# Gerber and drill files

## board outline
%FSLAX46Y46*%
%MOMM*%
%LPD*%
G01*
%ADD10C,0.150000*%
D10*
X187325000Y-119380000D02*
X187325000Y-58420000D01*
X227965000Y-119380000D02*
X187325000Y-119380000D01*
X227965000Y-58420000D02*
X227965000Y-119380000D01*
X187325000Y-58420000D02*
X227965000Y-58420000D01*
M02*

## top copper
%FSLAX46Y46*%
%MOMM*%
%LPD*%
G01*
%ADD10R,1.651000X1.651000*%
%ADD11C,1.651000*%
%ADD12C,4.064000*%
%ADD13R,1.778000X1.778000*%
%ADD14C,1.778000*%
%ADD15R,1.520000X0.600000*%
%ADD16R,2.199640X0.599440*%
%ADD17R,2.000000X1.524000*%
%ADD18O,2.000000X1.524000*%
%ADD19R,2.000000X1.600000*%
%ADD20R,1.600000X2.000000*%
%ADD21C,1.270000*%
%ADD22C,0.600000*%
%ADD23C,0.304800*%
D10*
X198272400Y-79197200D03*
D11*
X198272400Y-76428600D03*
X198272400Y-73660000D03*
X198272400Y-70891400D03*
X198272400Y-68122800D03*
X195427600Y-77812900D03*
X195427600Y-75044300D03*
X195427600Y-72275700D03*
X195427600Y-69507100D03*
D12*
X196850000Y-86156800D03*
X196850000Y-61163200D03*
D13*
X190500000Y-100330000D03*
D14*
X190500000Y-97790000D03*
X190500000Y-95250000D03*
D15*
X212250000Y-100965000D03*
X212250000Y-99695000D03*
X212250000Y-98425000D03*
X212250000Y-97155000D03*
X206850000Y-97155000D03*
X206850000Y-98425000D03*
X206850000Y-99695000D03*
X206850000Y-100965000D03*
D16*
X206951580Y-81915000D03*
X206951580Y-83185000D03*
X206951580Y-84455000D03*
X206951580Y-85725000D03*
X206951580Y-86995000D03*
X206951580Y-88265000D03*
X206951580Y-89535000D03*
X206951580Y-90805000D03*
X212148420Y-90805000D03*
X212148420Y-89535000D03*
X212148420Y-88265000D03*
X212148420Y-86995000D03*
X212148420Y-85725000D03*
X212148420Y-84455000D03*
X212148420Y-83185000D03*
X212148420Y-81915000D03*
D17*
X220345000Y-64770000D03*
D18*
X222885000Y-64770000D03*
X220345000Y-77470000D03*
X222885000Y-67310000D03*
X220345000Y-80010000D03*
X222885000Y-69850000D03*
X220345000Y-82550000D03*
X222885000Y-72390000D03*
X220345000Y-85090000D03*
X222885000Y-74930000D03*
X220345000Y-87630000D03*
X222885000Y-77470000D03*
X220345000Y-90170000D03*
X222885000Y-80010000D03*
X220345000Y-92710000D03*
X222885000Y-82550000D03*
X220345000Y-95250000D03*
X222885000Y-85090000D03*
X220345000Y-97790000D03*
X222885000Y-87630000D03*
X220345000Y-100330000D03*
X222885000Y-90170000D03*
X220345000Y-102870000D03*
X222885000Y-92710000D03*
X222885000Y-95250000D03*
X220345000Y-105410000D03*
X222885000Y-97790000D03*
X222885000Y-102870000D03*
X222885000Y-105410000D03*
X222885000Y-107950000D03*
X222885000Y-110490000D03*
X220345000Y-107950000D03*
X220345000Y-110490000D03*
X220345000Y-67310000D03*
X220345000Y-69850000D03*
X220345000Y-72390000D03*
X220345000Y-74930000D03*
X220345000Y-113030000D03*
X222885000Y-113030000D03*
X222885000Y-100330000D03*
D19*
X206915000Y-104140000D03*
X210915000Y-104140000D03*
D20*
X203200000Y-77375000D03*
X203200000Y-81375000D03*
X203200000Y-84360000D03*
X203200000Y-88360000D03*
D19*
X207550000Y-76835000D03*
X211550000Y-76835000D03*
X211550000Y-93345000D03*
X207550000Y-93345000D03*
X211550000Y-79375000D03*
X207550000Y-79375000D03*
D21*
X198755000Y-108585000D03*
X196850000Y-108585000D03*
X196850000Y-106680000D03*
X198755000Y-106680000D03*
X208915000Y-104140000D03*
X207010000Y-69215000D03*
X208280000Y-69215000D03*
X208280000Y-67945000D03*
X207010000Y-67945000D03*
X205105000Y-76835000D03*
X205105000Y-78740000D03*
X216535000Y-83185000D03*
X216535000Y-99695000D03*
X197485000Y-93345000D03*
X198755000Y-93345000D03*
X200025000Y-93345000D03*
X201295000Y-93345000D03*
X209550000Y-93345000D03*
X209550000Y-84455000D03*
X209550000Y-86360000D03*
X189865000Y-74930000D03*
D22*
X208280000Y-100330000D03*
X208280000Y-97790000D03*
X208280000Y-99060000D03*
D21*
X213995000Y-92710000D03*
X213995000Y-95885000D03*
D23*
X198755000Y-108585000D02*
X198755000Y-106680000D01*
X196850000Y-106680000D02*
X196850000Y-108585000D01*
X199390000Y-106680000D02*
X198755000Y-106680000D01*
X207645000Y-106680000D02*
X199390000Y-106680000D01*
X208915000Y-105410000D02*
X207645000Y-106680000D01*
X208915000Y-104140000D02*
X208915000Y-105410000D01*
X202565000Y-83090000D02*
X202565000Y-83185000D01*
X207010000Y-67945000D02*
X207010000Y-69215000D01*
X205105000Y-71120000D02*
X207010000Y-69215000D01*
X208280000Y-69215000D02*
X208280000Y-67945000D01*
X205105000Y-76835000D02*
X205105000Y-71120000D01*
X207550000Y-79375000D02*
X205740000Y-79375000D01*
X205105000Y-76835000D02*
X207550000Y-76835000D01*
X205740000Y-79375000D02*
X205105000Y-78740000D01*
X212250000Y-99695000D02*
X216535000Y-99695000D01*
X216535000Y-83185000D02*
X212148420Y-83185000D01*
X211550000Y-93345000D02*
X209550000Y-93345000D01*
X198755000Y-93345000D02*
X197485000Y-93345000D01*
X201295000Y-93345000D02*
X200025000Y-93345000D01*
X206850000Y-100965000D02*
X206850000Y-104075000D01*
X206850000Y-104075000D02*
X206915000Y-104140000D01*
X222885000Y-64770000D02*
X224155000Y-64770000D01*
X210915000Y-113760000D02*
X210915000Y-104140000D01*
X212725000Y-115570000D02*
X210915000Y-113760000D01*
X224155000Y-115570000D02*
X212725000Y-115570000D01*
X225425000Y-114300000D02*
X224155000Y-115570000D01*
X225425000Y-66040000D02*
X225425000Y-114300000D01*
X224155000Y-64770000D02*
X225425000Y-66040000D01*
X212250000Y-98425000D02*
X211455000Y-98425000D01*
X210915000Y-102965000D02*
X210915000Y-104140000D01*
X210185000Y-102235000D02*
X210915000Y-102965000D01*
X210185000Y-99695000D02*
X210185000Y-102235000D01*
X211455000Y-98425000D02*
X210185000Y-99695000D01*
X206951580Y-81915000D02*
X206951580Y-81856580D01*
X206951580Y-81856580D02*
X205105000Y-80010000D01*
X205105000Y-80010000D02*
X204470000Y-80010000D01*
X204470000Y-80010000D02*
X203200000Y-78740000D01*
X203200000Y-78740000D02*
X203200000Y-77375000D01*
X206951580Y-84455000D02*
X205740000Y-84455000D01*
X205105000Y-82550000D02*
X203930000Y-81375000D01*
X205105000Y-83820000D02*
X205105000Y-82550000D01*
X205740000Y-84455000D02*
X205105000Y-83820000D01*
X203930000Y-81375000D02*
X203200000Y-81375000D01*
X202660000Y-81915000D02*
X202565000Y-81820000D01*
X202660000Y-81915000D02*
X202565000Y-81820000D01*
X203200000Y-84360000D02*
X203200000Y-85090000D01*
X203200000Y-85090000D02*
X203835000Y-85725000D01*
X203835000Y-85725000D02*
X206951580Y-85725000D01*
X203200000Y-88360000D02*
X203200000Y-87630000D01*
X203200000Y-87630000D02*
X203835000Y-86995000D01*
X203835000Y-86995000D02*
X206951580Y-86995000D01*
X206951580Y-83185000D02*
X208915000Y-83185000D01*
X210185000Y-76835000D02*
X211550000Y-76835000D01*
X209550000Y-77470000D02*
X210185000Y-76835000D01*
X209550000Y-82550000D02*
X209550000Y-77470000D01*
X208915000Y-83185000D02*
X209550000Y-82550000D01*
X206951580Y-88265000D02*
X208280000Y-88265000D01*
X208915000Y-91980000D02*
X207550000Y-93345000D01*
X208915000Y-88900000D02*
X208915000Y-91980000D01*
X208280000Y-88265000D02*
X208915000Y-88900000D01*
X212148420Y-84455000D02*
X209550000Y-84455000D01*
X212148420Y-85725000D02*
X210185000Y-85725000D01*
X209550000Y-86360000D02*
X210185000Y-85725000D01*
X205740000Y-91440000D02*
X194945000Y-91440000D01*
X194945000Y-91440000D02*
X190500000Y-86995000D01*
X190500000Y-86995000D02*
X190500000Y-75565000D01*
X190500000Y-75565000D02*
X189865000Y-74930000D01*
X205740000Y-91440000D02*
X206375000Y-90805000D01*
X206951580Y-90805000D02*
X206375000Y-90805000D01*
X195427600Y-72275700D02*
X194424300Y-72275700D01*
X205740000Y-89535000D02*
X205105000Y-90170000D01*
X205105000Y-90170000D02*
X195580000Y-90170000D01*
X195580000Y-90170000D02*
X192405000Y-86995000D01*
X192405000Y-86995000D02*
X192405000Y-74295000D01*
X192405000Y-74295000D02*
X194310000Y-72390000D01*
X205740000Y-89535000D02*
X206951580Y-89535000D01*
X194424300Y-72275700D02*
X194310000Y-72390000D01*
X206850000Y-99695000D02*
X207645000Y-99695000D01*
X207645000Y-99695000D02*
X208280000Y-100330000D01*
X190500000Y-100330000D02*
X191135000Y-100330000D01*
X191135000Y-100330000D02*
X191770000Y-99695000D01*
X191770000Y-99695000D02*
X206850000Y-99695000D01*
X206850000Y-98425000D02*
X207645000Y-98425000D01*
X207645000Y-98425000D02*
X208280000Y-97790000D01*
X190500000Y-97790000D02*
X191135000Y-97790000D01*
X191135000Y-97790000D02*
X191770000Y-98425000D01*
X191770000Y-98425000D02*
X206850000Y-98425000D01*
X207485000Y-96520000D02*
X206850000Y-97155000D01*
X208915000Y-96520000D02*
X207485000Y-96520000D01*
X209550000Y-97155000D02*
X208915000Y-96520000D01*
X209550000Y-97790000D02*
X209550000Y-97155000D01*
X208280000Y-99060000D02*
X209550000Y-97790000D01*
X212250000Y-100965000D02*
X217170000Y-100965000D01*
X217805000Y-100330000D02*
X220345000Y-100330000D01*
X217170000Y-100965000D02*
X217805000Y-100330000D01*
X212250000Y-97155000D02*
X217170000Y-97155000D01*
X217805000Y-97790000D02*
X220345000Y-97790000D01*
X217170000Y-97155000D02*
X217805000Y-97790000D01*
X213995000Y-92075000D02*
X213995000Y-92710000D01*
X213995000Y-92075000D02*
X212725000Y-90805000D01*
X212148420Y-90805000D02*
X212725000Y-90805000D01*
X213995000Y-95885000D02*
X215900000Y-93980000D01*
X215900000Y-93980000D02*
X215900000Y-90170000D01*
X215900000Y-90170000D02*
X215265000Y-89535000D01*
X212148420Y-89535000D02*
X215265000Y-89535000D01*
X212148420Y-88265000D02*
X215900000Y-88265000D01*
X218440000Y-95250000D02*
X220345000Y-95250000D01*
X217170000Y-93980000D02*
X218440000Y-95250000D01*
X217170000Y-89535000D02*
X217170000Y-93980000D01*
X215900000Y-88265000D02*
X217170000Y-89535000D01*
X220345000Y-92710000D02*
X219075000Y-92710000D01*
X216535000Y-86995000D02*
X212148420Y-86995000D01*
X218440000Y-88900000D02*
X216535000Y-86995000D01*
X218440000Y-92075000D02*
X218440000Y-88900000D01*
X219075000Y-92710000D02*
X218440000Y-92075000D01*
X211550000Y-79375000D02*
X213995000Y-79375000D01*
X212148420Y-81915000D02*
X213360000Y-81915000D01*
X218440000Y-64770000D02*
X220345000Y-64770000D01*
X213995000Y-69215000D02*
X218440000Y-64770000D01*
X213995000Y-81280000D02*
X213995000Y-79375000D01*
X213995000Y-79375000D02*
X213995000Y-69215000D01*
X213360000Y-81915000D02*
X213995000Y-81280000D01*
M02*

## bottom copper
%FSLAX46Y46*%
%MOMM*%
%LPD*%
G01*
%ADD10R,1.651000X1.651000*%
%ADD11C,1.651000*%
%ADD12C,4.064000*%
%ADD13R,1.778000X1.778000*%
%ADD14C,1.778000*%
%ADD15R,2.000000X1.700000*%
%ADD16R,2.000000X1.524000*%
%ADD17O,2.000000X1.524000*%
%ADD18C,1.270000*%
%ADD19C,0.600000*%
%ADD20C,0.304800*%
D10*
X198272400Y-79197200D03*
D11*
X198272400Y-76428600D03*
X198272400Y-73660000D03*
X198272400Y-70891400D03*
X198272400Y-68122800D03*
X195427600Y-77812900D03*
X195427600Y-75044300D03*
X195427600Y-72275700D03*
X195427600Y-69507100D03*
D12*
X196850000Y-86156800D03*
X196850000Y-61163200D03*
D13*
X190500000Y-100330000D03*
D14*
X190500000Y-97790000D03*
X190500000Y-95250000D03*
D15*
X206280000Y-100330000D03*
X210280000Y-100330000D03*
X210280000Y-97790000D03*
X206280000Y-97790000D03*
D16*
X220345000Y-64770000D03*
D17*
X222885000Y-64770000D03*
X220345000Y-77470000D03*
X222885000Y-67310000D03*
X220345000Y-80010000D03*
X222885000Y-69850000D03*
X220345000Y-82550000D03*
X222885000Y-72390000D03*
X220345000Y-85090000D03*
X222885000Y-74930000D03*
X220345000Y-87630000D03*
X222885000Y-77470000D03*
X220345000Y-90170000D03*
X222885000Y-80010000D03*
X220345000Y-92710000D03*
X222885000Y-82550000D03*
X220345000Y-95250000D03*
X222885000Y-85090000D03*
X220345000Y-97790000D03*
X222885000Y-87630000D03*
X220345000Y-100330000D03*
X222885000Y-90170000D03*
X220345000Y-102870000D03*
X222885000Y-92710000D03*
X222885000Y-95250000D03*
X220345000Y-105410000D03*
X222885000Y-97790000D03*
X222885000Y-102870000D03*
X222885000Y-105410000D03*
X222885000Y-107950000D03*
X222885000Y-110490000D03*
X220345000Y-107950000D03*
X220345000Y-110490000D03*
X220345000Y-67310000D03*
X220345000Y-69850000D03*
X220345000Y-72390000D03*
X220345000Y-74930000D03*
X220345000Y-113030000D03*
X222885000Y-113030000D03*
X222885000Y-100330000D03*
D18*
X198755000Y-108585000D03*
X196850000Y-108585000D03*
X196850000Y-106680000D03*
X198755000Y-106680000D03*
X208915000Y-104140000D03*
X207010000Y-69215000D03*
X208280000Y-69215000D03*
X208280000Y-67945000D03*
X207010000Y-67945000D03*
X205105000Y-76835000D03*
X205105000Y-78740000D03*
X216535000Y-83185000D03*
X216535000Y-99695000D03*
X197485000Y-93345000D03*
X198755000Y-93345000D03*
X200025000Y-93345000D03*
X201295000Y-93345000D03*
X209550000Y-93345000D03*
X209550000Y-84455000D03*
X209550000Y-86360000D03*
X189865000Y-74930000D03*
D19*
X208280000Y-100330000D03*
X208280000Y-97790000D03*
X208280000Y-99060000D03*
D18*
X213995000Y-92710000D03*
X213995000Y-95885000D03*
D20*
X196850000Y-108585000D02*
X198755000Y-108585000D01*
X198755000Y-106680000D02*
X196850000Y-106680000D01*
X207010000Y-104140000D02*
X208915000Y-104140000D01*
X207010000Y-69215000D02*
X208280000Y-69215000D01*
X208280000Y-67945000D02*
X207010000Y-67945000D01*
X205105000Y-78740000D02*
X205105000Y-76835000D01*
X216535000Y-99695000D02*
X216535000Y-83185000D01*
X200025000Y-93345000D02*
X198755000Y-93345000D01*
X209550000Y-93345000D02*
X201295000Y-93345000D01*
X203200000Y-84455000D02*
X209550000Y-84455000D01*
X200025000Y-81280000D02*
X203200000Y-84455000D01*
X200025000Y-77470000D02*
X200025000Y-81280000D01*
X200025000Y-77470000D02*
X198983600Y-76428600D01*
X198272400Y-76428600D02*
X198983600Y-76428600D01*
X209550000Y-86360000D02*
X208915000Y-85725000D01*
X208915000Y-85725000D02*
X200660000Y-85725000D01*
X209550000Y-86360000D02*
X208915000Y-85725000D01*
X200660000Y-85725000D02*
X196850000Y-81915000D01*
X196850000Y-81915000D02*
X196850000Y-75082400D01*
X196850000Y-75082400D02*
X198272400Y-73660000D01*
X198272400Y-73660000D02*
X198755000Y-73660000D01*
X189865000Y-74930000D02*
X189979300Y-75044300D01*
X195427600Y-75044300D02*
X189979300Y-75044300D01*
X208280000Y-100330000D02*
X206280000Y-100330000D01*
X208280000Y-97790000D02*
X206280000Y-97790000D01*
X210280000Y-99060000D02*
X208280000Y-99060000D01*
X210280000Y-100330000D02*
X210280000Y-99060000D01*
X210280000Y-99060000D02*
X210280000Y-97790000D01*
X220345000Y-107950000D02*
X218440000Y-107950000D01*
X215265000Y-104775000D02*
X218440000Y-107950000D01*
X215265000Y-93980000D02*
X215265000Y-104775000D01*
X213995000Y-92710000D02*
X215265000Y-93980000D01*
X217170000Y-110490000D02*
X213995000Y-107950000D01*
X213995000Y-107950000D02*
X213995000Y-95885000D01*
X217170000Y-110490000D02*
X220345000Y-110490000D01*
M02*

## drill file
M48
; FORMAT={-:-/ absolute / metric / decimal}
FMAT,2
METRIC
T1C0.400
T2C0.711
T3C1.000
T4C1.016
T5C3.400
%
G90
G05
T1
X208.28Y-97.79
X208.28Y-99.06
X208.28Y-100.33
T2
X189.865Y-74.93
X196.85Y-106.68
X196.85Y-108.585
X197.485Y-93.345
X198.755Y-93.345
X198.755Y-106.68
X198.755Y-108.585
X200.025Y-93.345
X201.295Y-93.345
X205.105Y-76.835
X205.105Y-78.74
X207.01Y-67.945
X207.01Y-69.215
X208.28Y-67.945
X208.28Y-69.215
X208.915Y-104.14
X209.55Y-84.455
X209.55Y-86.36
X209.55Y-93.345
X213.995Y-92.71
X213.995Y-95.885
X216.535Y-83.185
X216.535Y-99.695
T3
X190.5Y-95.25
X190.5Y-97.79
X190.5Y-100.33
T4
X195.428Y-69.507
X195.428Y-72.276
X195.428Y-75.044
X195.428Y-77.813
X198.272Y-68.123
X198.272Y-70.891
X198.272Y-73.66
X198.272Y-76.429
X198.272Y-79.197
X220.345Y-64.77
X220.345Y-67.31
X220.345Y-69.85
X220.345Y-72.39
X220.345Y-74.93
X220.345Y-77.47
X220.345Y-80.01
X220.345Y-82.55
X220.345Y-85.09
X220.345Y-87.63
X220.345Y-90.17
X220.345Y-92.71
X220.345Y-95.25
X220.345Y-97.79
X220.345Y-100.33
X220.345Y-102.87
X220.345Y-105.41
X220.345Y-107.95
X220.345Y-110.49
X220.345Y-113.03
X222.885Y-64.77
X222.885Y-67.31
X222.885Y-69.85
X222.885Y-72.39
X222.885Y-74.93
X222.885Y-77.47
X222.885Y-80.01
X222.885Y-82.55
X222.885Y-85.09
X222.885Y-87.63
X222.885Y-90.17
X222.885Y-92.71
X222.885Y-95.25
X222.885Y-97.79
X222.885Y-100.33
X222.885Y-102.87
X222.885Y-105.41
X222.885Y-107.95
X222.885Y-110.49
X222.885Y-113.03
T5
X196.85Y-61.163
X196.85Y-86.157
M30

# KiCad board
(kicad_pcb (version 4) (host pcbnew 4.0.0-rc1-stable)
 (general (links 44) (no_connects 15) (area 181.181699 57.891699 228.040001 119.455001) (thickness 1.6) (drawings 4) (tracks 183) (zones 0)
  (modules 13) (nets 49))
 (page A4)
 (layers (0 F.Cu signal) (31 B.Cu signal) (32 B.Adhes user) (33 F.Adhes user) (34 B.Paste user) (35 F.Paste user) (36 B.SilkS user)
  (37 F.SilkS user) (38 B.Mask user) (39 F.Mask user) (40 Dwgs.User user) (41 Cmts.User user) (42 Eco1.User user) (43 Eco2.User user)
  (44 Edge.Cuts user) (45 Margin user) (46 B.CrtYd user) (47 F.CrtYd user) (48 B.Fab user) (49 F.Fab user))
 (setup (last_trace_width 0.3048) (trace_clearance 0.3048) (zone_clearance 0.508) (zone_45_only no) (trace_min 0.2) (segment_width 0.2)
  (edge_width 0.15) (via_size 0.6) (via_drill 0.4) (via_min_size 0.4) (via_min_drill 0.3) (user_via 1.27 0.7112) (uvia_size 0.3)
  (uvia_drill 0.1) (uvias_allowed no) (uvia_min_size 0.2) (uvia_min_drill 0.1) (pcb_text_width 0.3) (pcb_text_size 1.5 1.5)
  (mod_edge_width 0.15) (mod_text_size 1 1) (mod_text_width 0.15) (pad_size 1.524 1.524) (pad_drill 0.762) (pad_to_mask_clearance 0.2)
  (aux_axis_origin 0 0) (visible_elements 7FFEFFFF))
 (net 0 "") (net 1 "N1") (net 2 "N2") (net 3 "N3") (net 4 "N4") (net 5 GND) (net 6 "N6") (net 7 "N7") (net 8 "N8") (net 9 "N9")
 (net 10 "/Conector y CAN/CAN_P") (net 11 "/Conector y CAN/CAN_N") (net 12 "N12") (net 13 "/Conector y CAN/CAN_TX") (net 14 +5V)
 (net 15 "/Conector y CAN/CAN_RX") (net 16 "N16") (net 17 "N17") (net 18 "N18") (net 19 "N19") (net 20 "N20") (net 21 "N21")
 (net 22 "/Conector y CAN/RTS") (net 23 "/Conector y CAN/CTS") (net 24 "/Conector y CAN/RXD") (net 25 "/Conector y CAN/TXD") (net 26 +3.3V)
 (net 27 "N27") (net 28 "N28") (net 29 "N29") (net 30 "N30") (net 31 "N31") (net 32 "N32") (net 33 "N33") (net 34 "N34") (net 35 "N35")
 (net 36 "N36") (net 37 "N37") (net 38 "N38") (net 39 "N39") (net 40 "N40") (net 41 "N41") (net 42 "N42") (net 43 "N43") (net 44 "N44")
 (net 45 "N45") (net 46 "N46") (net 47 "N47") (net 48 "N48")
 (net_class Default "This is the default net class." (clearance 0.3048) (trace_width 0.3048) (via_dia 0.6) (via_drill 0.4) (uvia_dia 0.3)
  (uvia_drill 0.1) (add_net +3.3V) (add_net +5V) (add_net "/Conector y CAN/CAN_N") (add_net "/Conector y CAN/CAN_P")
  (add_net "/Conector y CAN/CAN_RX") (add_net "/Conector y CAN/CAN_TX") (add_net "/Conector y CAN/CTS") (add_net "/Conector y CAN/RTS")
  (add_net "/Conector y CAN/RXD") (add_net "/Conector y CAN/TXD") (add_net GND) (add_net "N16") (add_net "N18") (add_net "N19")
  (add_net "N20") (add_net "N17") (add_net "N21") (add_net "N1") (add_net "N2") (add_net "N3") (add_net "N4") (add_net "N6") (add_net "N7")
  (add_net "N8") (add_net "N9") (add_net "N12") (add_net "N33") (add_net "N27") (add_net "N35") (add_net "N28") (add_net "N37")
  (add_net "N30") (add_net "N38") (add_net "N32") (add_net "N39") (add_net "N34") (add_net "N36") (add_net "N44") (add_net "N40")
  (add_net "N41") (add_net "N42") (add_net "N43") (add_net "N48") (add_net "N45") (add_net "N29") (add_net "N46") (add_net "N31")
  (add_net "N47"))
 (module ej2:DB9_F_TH (layer F.Cu) (at 196.85 73.66 90)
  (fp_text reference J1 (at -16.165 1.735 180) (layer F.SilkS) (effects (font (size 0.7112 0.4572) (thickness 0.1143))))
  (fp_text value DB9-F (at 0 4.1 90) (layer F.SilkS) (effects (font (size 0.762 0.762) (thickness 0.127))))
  (pad 1 thru_hole rect (at -5.5372 1.4224 90) (size 1.651 1.651) (drill 1.016) (layers *.Cu *.Mask) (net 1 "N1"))
  (pad 2 thru_hole circle (at -2.7686 1.4224 90) (size 1.651 1.651) (drill 1.016) (layers *.Cu *.Mask) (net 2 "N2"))
  (pad 3 thru_hole circle (at 0 1.4224 90) (size 1.651 1.651) (drill 1.016) (layers *.Cu *.Mask) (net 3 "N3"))
  (pad 4 thru_hole circle (at 2.7686 1.4224 90) (size 1.651 1.651) (drill 1.016) (layers *.Cu *.Mask) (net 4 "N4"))
  (pad 5 thru_hole circle (at 5.5372 1.4224 90) (size 1.651 1.651) (drill 1.016) (layers *.Cu *.Mask) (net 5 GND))
  (pad 6 thru_hole circle (at -4.1529 -1.4224 90) (size 1.651 1.651) (drill 1.016) (layers *.Cu *.Mask) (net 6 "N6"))
  (pad 7 thru_hole circle (at -1.3843 -1.4224 90) (size 1.651 1.651) (drill 1.016) (layers *.Cu *.Mask) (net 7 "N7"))
  (pad 8 thru_hole circle (at 1.3843 -1.4224 90) (size 1.651 1.651) (drill 1.016) (layers *.Cu *.Mask) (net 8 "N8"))
  (pad 9 thru_hole circle (at 4.1529 -1.4224 90) (size 1.651 1.651) (drill 1.016) (layers *.Cu *.Mask) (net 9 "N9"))
  (pad 10 thru_hole circle (at -12.4968 0 90) (size 4.064 4.064) (drill 3.4) (layers *.Cu *.Mask))
  (pad 11 thru_hole circle (at 12.4968 0 90) (size 4.064 4.064) (drill 3.4) (layers *.Cu *.Mask)))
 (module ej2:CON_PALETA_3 (layer F.Cu) (at 190.5 97.79 90)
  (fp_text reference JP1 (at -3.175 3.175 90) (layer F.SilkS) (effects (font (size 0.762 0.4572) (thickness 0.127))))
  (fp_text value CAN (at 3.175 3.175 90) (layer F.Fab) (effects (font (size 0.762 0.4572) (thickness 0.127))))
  (pad 1 thru_hole rect (at -2.54 0 90) (size 1.778 1.778) (drill 1) (layers *.Cu *.Mask) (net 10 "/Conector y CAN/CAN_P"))
  (pad 2 thru_hole circle (at 0 0 90) (size 1.778 1.778) (drill 1) (layers *.Cu *.Mask) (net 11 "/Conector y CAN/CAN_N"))
  (pad 3 thru_hole circle (at 2.54 0 90) (size 1.778 1.778) (drill 1) (layers *.Cu *.Mask) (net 5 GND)))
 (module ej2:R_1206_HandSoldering (layer B.Cu) (at 208.28 100.33)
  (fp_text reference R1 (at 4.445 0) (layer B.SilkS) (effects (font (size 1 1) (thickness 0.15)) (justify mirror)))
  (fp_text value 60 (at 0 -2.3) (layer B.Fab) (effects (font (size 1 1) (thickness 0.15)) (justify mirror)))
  (pad 1 smd rect (at -2 0) (size 2 1.7) (layers B.Cu B.Paste B.Mask) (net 10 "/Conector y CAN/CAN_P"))
  (pad 2 smd rect (at 2 0) (size 2 1.7) (layers B.Cu B.Paste B.Mask) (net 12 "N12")))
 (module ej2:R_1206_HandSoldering (layer B.Cu) (at 208.28 97.79 180)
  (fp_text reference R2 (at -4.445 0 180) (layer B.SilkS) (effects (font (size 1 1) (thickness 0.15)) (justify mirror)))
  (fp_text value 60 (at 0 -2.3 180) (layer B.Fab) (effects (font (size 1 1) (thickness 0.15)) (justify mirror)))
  (pad 1 smd rect (at -2 0 180) (size 2 1.7) (layers B.Cu B.Paste B.Mask) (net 12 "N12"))
  (pad 2 smd rect (at 2 0 180) (size 2 1.7) (layers B.Cu B.Paste B.Mask) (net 11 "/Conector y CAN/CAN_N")))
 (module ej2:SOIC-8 (layer F.Cu) (at 209.55 99.06 180)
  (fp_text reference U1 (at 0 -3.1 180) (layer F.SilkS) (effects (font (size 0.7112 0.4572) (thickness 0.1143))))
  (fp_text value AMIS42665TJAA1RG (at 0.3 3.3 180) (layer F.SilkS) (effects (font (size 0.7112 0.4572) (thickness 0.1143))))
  (pad 1 smd rect (at -2.7 -1.905 90) (size 0.6 1.52) (layers F.Cu F.Paste F.Mask) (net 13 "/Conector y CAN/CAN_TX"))
  (pad 2 smd rect (at -2.7 -0.635 90) (size 0.6 1.52) (layers F.Cu F.Paste F.Mask) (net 5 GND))
  (pad 3 smd rect (at -2.7 0.635 90) (size 0.6 1.52) (layers F.Cu F.Paste F.Mask) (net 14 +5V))
  (pad 4 smd rect (at -2.7 1.905 90) (size 0.6 1.52) (layers F.Cu F.Paste F.Mask) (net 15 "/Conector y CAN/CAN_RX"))
  (pad 5 smd rect (at 2.7 1.905 90) (size 0.6 1.52) (layers F.Cu F.Paste F.Mask) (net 12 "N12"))
  (pad 6 smd rect (at 2.7 0.635 90) (size 0.6 1.52) (layers F.Cu F.Paste F.Mask) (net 11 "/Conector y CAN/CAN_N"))
  (pad 7 smd rect (at 2.7 -0.635 90) (size 0.6 1.52) (layers F.Cu F.Paste F.Mask) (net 10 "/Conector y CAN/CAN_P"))
  (pad 8 smd rect (at 2.7 -1.905 90) (size 0.6 1.52) (layers F.Cu F.Paste F.Mask) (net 5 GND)))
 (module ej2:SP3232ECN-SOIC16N (layer F.Cu) (at 209.55 86.36 270)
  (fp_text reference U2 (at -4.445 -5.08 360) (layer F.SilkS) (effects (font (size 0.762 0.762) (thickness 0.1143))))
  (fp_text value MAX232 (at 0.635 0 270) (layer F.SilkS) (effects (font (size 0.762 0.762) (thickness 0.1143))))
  (pad 1 smd rect (at -4.445 2.59842 270) (size 0.59944 2.19964) (layers F.Cu F.Paste F.Mask) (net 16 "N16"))
  (pad 2 smd rect (at -3.175 2.59842 270) (size 0.59944 2.19964) (layers F.Cu F.Paste F.Mask) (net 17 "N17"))
  (pad 3 smd rect (at -1.905 2.59842 270) (size 0.59944 2.19964) (layers F.Cu F.Paste F.Mask) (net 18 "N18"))
  (pad 4 smd rect (at -0.635 2.59842 270) (size 0.59944 2.19964) (layers F.Cu F.Paste F.Mask) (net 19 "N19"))
  (pad 5 smd rect (at 0.635 2.59842 270) (size 0.59944 2.19964) (layers F.Cu F.Paste F.Mask) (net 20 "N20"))
  (pad 6 smd rect (at 1.905 2.59842 270) (size 0.59944 2.19964) (layers F.Cu F.Paste F.Mask) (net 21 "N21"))
  (pad 7 smd rect (at 3.175 2.59842 270) (size 0.59944 2.19964) (layers F.Cu F.Paste F.Mask) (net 8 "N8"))
  (pad 8 smd rect (at 4.445 2.59842 270) (size 0.59944 2.19964) (layers F.Cu F.Paste F.Mask) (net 7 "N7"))
  (pad 9 smd rect (at 4.445 -2.59842 270) (size 0.59944 2.19964) (layers F.Cu F.Paste F.Mask) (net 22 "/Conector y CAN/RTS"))
  (pad 10 smd rect (at 3.175 -2.59842 270) (size 0.59944 2.19964) (layers F.Cu F.Paste F.Mask) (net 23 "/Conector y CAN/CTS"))
  (pad 11 smd rect (at 1.905 -2.59842 270) (size 0.59944 2.19964) (layers F.Cu F.Paste F.Mask) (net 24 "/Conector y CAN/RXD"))
  (pad 12 smd rect (at 0.635 -2.59842 270) (size 0.59944 2.19964) (layers F.Cu F.Paste F.Mask) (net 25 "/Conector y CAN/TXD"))
  (pad 13 smd rect (at -0.635 -2.59842 270) (size 0.59944 2.19964) (layers F.Cu F.Paste F.Mask) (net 3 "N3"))
  (pad 14 smd rect (at -1.905 -2.59842 270) (size 0.59944 2.19964) (layers F.Cu F.Paste F.Mask) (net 2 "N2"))
  (pad 15 smd rect (at -3.175 -2.59842 270) (size 0.59944 2.19964) (layers F.Cu F.Paste F.Mask) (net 5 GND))
  (pad 16 smd rect (at -4.445 -2.59842 270) (size 0.59944 2.19964) (layers F.Cu F.Paste F.Mask) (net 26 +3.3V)))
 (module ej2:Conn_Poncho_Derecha (layer F.Cu) (at 220.345 64.77)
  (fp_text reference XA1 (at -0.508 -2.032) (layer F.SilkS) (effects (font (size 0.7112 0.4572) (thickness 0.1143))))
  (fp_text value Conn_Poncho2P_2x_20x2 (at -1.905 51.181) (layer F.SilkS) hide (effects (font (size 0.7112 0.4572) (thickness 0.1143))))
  (pad 1 thru_hole rect (at 0 0 270) (size 1.524 2) (drill 1.016) (layers *.Cu *.Mask) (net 26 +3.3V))
  (pad 2 thru_hole oval (at 2.54 0 270) (size 1.524 2) (drill 1.016) (layers *.Cu *.Mask) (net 14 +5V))
  (pad 11 thru_hole oval (at 0 12.7 270) (size 1.524 2) (drill 1.016) (layers *.Cu *.Mask) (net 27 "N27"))
  (pad 4 thru_hole oval (at 2.54 2.54 270) (size 1.524 2) (drill 1.016) (layers *.Cu *.Mask) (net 5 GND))
  (pad 13 thru_hole oval (at 0 15.24 270) (size 1.524 2) (drill 1.016) (layers *.Cu *.Mask) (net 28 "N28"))
  (pad 6 thru_hole oval (at 2.54 5.08 270) (size 1.524 2) (drill 1.016) (layers *.Cu *.Mask) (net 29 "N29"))
  (pad 15 thru_hole oval (at 0 17.78 270) (size 1.524 2) (drill 1.016) (layers *.Cu *.Mask) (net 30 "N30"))
  (pad 8 thru_hole oval (at 2.54 7.62 270) (size 1.524 2) (drill 1.016) (layers *.Cu *.Mask) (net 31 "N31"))
  (pad 17 thru_hole oval (at 0 20.32 270) (size 1.524 2) (drill 1.016) (layers *.Cu *.Mask) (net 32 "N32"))
  (pad 10 thru_hole oval (at 2.54 10.16 270) (size 1.524 2) (drill 1.016) (layers *.Cu *.Mask) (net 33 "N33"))
  (pad 19 thru_hole oval (at 0 22.86 270) (size 1.524 2) (drill 1.016) (layers *.Cu *.Mask) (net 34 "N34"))
  (pad 12 thru_hole oval (at 2.54 12.7 270) (size 1.524 2) (drill 1.016) (layers *.Cu *.Mask) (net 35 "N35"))
  (pad 21 thru_hole oval (at 0 25.4 270) (size 1.524 2) (drill 1.016) (layers *.Cu *.Mask) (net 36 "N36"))
  (pad 14 thru_hole oval (at 2.54 15.24 270) (size 1.524 2) (drill 1.016) (layers *.Cu *.Mask) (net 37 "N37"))
  (pad 23 thru_hole oval (at 0 27.94 270) (size 1.524 2) (drill 1.016) (layers *.Cu *.Mask) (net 25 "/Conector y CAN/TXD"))
  (pad 16 thru_hole oval (at 2.54 17.78 270) (size 1.524 2) (drill 1.016) (layers *.Cu *.Mask) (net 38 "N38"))
  (pad 25 thru_hole oval (at 0 30.48 270) (size 1.524 2) (drill 1.016) (layers *.Cu *.Mask) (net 24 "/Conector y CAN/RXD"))
  (pad 18 thru_hole oval (at 2.54 20.32 270) (size 1.524 2) (drill 1.016) (layers *.Cu *.Mask) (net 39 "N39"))
  (pad 27 thru_hole oval (at 0 33.02 270) (size 1.524 2) (drill 1.016) (layers *.Cu *.Mask) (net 15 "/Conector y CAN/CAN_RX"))
  (pad 20 thru_hole oval (at 2.54 22.86 270) (size 1.524 2) (drill 1.016) (layers *.Cu *.Mask) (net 5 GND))
  (pad 29 thru_hole oval (at 0 35.56 270) (size 1.524 2) (drill 1.016) (layers *.Cu *.Mask) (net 13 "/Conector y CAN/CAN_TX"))
  (pad 22 thru_hole oval (at 2.54 25.4 270) (size 1.524 2) (drill 1.016) (layers *.Cu *.Mask) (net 5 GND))
  (pad 31 thru_hole oval (at 0 38.1 270) (size 1.524 2) (drill 1.016) (layers *.Cu *.Mask) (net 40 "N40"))
  (pad 24 thru_hole oval (at 2.54 27.94 270) (size 1.524 2) (drill 1.016) (layers *.Cu *.Mask) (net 5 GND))
  (pad 26 thru_hole oval (at 2.54 30.48 270) (size 1.524 2) (drill 1.016) (layers *.Cu *.Mask) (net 5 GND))
  (pad 33 thru_hole oval (at 0 40.64 270) (size 1.524 2) (drill 1.016) (layers *.Cu *.Mask) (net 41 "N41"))
  (pad 28 thru_hole oval (at 2.54 33.02 270) (size 1.524 2) (drill 1.016) (layers *.Cu *.Mask) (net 5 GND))
  (pad 32 thru_hole oval (at 2.54 38.1 270) (size 1.524 2) (drill 1.016) (layers *.Cu *.Mask) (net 5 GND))
  (pad 34 thru_hole oval (at 2.54 40.64 270) (size 1.524 2) (drill 1.016) (layers *.Cu *.Mask) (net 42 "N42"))
  (pad 36 thru_hole oval (at 2.54 43.18 270) (size 1.524 2) (drill 1.016) (layers *.Cu *.Mask) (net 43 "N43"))
  (pad 38 thru_hole oval (at 2.54 45.72 270) (size 1.524 2) (drill 1.016) (layers *.Cu *.Mask) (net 5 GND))
  (pad 35 thru_hole oval (at 0 43.18 270) (size 1.524 2) (drill 1.016) (layers *.Cu *.Mask) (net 22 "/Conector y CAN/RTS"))
  (pad 37 thru_hole oval (at 0 45.72 270) (size 1.524 2) (drill 1.016) (layers *.Cu *.Mask) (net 23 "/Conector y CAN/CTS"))
  (pad 3 thru_hole oval (at 0 2.54 270) (size 1.524 2) (drill 1.016) (layers *.Cu *.Mask) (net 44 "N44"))
  (pad 5 thru_hole oval (at 0 5.08 270) (size 1.524 2) (drill 1.016) (layers *.Cu *.Mask) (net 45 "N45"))
  (pad 7 thru_hole oval (at 0 7.62 270) (size 1.524 2) (drill 1.016) (layers *.Cu *.Mask) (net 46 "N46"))
  (pad 9 thru_hole oval (at 0 10.16 270) (size 1.524 2) (drill 1.016) (layers *.Cu *.Mask) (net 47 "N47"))
  (pad 39 thru_hole oval (at 0 48.26 270) (size 1.524 2) (drill 1.016) (layers *.Cu *.Mask) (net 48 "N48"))
  (pad 40 thru_hole oval (at 2.54 48.26 270) (size 1.524 2) (drill 1.016) (layers *.Cu *.Mask) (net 5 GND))
  (pad 30 thru_hole oval (at 2.54 35.56 270) (size 1.524 2) (drill 1.016) (layers *.Cu *.Mask) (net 5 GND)))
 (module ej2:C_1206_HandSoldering (layer F.Cu) (at 208.915 104.14)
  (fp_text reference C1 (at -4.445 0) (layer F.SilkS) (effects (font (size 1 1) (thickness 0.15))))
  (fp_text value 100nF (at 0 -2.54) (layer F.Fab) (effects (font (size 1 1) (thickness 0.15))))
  (pad 1 smd rect (at -2 0) (size 2 1.6) (layers F.Cu F.Paste F.Mask) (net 5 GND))
  (pad 2 smd rect (at 2 0) (size 2 1.6) (layers F.Cu F.Paste F.Mask) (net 14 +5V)))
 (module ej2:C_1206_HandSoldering (layer F.Cu) (at 203.2 79.375 270)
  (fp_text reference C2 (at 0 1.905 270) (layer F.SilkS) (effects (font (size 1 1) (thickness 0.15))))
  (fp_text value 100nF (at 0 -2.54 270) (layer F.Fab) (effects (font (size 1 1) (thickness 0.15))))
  (pad 1 smd rect (at -2 0 270) (size 2 1.6) (layers F.Cu F.Paste F.Mask) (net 16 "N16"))
  (pad 2 smd rect (at 2 0 270) (size 2 1.6) (layers F.Cu F.Paste F.Mask) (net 18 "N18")))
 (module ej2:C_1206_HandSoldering (layer F.Cu) (at 203.2 86.36 270)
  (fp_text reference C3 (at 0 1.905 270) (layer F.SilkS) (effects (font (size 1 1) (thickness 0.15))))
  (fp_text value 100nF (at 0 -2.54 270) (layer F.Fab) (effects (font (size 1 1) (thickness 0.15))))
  (pad 1 smd rect (at -2 0 270) (size 2 1.6) (layers F.Cu F.Paste F.Mask) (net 19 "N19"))
  (pad 2 smd rect (at 2 0 270) (size 2 1.6) (layers F.Cu F.Paste F.Mask) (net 20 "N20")))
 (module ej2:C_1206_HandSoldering (layer F.Cu) (at 209.55 76.835)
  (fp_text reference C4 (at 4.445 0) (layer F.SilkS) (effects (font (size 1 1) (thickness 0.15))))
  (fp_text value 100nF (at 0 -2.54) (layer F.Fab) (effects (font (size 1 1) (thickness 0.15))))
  (pad 1 smd rect (at -2 0) (size 2 1.6) (layers F.Cu F.Paste F.Mask) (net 5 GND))
  (pad 2 smd rect (at 2 0) (size 2 1.6) (layers F.Cu F.Paste F.Mask) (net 17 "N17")))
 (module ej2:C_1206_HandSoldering (layer F.Cu) (at 209.55 93.345 180)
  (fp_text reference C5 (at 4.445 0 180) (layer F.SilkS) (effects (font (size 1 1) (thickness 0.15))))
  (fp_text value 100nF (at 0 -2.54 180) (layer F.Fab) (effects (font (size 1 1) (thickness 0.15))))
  (pad 1 smd rect (at -2 0 180) (size 2 1.6) (layers F.Cu F.Paste F.Mask) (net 5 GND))
  (pad 2 smd rect (at 2 0 180) (size 2 1.6) (layers F.Cu F.Paste F.Mask) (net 21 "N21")))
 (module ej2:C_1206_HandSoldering (layer F.Cu) (at 209.55 79.375 180)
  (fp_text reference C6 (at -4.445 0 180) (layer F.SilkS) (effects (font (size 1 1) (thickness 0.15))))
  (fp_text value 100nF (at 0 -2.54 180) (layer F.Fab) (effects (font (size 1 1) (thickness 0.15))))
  (pad 1 smd rect (at -2 0 180) (size 2 1.6) (layers F.Cu F.Paste F.Mask) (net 26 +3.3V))
  (pad 2 smd rect (at 2 0 180) (size 2 1.6) (layers F.Cu F.Paste F.Mask) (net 5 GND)))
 (gr_line (start 187.325 119.38) (end 187.325 58.42) (angle 90) (layer Edge.Cuts) (width 0.15))
 (gr_line (start 227.965 119.38) (end 187.325 119.38) (angle 90) (layer Edge.Cuts) (width 0.15))
 (gr_line (start 227.965 58.42) (end 227.965 119.38) (angle 90) (layer Edge.Cuts) (width 0.15))
 (gr_line (start 187.325 58.42) (end 227.965 58.42) (angle 90) (layer Edge.Cuts) (width 0.15))
 (segment (start 198.755 108.585) (end 198.755 106.68) (width 0.3048) (layer F.Cu) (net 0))
 (via (at 198.755 108.585) (size 1.27) (drill 0.7112) (layers F.Cu B.Cu) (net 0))
 (segment (start 196.85 108.585) (end 198.755 108.585) (width 0.3048) (layer B.Cu) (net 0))
 (via (at 196.85 108.585) (size 1.27) (drill 0.7112) (layers F.Cu B.Cu) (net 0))
 (segment (start 196.85 106.68) (end 196.85 108.585) (width 0.3048) (layer F.Cu) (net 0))
 (via (at 196.85 106.68) (size 1.27) (drill 0.7112) (layers F.Cu B.Cu) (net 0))
 (segment (start 198.755 106.68) (end 196.85 106.68) (width 0.3048) (layer B.Cu) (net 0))
 (via (at 198.755 106.68) (size 1.27) (drill 0.7112) (layers F.Cu B.Cu) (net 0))
 (segment (start 199.39 106.68) (end 198.755 106.68) (width 0.3048) (layer F.Cu) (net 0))
 (segment (start 207.645 106.68) (end 199.39 106.68) (width 0.3048) (layer F.Cu) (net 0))
 (segment (start 208.915 105.41) (end 207.645 106.68) (width 0.3048) (layer F.Cu) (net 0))
 (segment (start 208.915 104.14) (end 208.915 105.41) (width 0.3048) (layer F.Cu) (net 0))
 (via (at 208.915 104.14) (size 1.27) (drill 0.7112) (layers F.Cu B.Cu) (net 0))
 (segment (start 207.01 104.14) (end 208.915 104.14) (width 0.3048) (layer B.Cu) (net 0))
 (segment (start 202.565 83.09) (end 202.565 83.185) (width 0.3048) (layer F.Cu) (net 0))
 (segment (start 207.01 67.945) (end 207.01 69.215) (width 0.3048) (layer F.Cu) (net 5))
 (segment (start 205.105 71.12) (end 207.01 69.215) (width 0.3048) (layer F.Cu) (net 5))
 (via (at 207.01 69.215) (size 1.27) (drill 0.7112) (layers F.Cu B.Cu) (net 5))
 (segment (start 207.01 69.215) (end 208.28 69.215) (width 0.3048) (layer B.Cu) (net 5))
 (via (at 208.28 69.215) (size 1.27) (drill 0.7112) (layers F.Cu B.Cu) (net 5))
 (segment (start 208.28 69.215) (end 208.28 67.945) (width 0.3048) (layer F.Cu) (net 5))
 (via (at 208.28 67.945) (size 1.27) (drill 0.7112) (layers F.Cu B.Cu) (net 5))
 (segment (start 208.28 67.945) (end 207.01 67.945) (width 0.3048) (layer B.Cu) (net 5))
 (via (at 207.01 67.945) (size 1.27) (drill 0.7112) (layers F.Cu B.Cu) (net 5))
 (segment (start 205.105 76.835) (end 205.105 71.12) (width 0.3048) (layer F.Cu) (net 5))
 (segment (start 207.55 79.375) (end 205.74 79.375) (width 0.3048) (layer F.Cu) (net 5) (status 400000))
 (segment (start 205.105 76.835) (end 207.55 76.835) (width 0.3048) (layer F.Cu) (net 5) (status 800000))
 (via (at 205.105 76.835) (size 1.27) (drill 0.7112) (layers F.Cu B.Cu) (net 5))
 (segment (start 205.105 78.74) (end 205.105 76.835) (width 0.3048) (layer B.Cu) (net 5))
 (via (at 205.105 78.74) (size 1.27) (drill 0.7112) (layers F.Cu B.Cu) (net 5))
 (segment (start 205.74 79.375) (end 205.105 78.74) (width 0.3048) (layer F.Cu) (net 5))
 (segment (start 212.25 99.695) (end 216.535 99.695) (width 0.3048) (layer F.Cu) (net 5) (status 400000))
 (segment (start 216.535 83.185) (end 212.14842 83.185) (width 0.3048) (layer F.Cu) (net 5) (status 800000))
 (via (at 216.535 83.185) (size 1.27) (drill 0.7112) (layers F.Cu B.Cu) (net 5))
 (segment (start 216.535 99.695) (end 216.535 83.185) (width 0.3048) (layer B.Cu) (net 5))
 (via (at 216.535 99.695) (size 1.27) (drill 0.7112) (layers F.Cu B.Cu) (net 5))
 (segment (start 211.55 93.345) (end 209.55 93.345) (width 0.3048) (layer F.Cu) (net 5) (status 400000))
 (via (at 197.485 93.345) (size 1.27) (drill 0.7112) (layers F.Cu B.Cu) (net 5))
 (segment (start 198.755 93.345) (end 197.485 93.345) (width 0.3048) (layer F.Cu) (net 5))
 (via (at 198.755 93.345) (size 1.27) (drill 0.7112) (layers F.Cu B.Cu) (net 5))
 (segment (start 200.025 93.345) (end 198.755 93.345) (width 0.3048) (layer B.Cu) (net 5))
 (via (at 200.025 93.345) (size 1.27) (drill 0.7112) (layers F.Cu B.Cu) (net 5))
 (segment (start 201.295 93.345) (end 200.025 93.345) (width 0.3048) (layer F.Cu) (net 5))
 (via (at 201.295 93.345) (size 1.27) (drill 0.7112) (layers F.Cu B.Cu) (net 5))
 (segment (start 209.55 93.345) (end 201.295 93.345) (width 0.3048) (layer B.Cu) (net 5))
 (via (at 209.55 93.345) (size 1.27) (drill 0.7112) (layers F.Cu B.Cu) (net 5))
 (segment (start 206.85 100.965) (end 206.85 104.075) (width 0.3048) (layer F.Cu) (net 5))
 (segment (start 206.85 104.075) (end 206.915 104.14) (width 0.3048) (layer F.Cu) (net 5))
 (segment (start 222.885 64.77) (end 224.155 64.77) (width 0.3048) (layer F.Cu) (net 14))
 (segment (start 210.915 113.76) (end 210.915 104.14) (width 0.3048) (layer F.Cu) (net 14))
 (segment (start 212.725 115.57) (end 210.915 113.76) (width 0.3048) (layer F.Cu) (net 14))
 (segment (start 224.155 115.57) (end 212.725 115.57) (width 0.3048) (layer F.Cu) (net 14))
 (segment (start 225.425 114.3) (end 224.155 115.57) (width 0.3048) (layer F.Cu) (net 14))
 (segment (start 225.425 66.04) (end 225.425 114.3) (width 0.3048) (layer F.Cu) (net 14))
 (segment (start 224.155 64.77) (end 225.425 66.04) (width 0.3048) (layer F.Cu) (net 14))
 (segment (start 212.25 98.425) (end 211.455 98.425) (width 0.3048) (layer F.Cu) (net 14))
 (segment (start 210.915 102.965) (end 210.915 104.14) (width 0.3048) (layer F.Cu) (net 14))
 (segment (start 210.185 102.235) (end 210.915 102.965) (width 0.3048) (layer F.Cu) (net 14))
 (segment (start 210.185 99.695) (end 210.185 102.235) (width 0.3048) (layer F.Cu) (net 14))
 (segment (start 211.455 98.425) (end 210.185 99.695) (width 0.3048) (layer F.Cu) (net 14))
 (segment (start 206.95158 81.915) (end 206.95158 81.85658) (width 0.3048) (layer F.Cu) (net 16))
 (segment (start 206.95158 81.85658) (end 205.105 80.01) (width 0.3048) (layer F.Cu) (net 16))
 (segment (start 205.105 80.01) (end 204.47 80.01) (width 0.3048) (layer F.Cu) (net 16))
 (segment (start 204.47 80.01) (end 203.2 78.74) (width 0.3048) (layer F.Cu) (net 16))
 (segment (start 203.2 78.74) (end 203.2 77.375) (width 0.3048) (layer F.Cu) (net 16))
 (segment (start 206.95158 84.455) (end 205.74 84.455) (width 0.3048) (layer F.Cu) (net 18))
 (segment (start 205.105 82.55) (end 203.93 81.375) (width 0.3048) (layer F.Cu) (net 18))
 (segment (start 205.105 83.82) (end 205.105 82.55) (width 0.3048) (layer F.Cu) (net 18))
 (segment (start 205.74 84.455) (end 205.105 83.82) (width 0.3048) (layer F.Cu) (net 18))
 (segment (start 203.93 81.375) (end 203.2 81.375) (width 0.3048) (layer F.Cu) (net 18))
 (segment (start 202.66 81.915) (end 202.565 81.82) (width 0.3048) (layer F.Cu) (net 18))
 (segment (start 202.66 81.915) (end 202.565 81.82) (width 0.3048) (layer F.Cu) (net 18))
 (segment (start 203.2 84.36) (end 203.2 85.09) (width 0.3048) (layer F.Cu) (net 19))
 (segment (start 203.2 85.09) (end 203.835 85.725) (width 0.3048) (layer F.Cu) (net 19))
 (segment (start 203.835 85.725) (end 206.95158 85.725) (width 0.3048) (layer F.Cu) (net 19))
 (segment (start 203.2 88.36) (end 203.2 87.63) (width 0.3048) (layer F.Cu) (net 20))
 (segment (start 203.2 87.63) (end 203.835 86.995) (width 0.3048) (layer F.Cu) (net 20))
 (segment (start 203.835 86.995) (end 206.95158 86.995) (width 0.3048) (layer F.Cu) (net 20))
 (segment (start 206.95158 83.185) (end 208.915 83.185) (width 0.3048) (layer F.Cu) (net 17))
 (segment (start 210.185 76.835) (end 211.55 76.835) (width 0.3048) (layer F.Cu) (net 17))
 (segment (start 209.55 77.47) (end 210.185 76.835) (width 0.3048) (layer F.Cu) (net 17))
 (segment (start 209.55 82.55) (end 209.55 77.47) (width 0.3048) (layer F.Cu) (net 17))
 (segment (start 208.915 83.185) (end 209.55 82.55) (width 0.3048) (layer F.Cu) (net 17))
 (segment (start 206.95158 88.265) (end 208.28 88.265) (width 0.3048) (layer F.Cu) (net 21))
 (segment (start 208.915 91.98) (end 207.55 93.345) (width 0.3048) (layer F.Cu) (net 21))
 (segment (start 208.915 88.9) (end 208.915 91.98) (width 0.3048) (layer F.Cu) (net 21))
 (segment (start 208.28 88.265) (end 208.915 88.9) (width 0.3048) (layer F.Cu) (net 21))
 (via (at 209.55 84.455) (size 1.27) (drill 0.7112) (layers F.Cu B.Cu) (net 2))
 (segment (start 212.14842 84.455) (end 209.55 84.455) (width 0.3048) (layer F.Cu) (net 2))
 (segment (start 203.2 84.455) (end 209.55 84.455) (width 0.3048) (layer B.Cu) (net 2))
 (segment (start 200.025 81.28) (end 203.2 84.455) (width 0.3048) (layer B.Cu) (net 2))
 (segment (start 200.025 77.47) (end 200.025 81.28) (width 0.3048) (layer B.Cu) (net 2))
 (segment (start 200.025 77.47) (end 198.9836 76.4286) (width 0.3048) (layer B.Cu) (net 2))
 (segment (start 198.2724 76.4286) (end 198.9836 76.4286) (width 0.3048) (layer B.Cu) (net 2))
 (via (at 209.55 86.36) (size 1.27) (drill 0.7112) (layers F.Cu B.Cu) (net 3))
 (segment (start 209.55 86.36) (end 208.915 85.725) (width 0.3048) (layer B.Cu) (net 3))
 (segment (start 208.915 85.725) (end 200.66 85.725) (width 0.3048) (layer B.Cu) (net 3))
 (segment (start 212.14842 85.725) (end 210.185 85.725) (width 0.3048) (layer F.Cu) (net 3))
 (segment (start 209.55 86.36) (end 210.185 85.725) (width 0.3048) (layer F.Cu) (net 3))
 (segment (start 209.55 86.36) (end 208.915 85.725) (width 0.3048) (layer B.Cu) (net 3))
 (segment (start 200.66 85.725) (end 196.85 81.915) (width 0.3048) (layer B.Cu) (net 3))
 (segment (start 196.85 81.915) (end 196.85 75.0824) (width 0.3048) (layer B.Cu) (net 3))
 (segment (start 196.85 75.0824) (end 198.2724 73.66) (width 0.3048) (layer B.Cu) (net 3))
 (segment (start 198.2724 73.66) (end 198.755 73.66) (width 0.3048) (layer B.Cu) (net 3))
 (via (at 189.865 74.93) (size 1.27) (drill 0.7112) (layers F.Cu B.Cu) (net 7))
 (segment (start 205.74 91.44) (end 194.945 91.44) (width 0.3048) (layer F.Cu) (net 7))
 (segment (start 194.945 91.44) (end 190.5 86.995) (width 0.3048) (layer F.Cu) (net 7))
 (segment (start 190.5 86.995) (end 190.5 75.565) (width 0.3048) (layer F.Cu) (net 7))
 (segment (start 190.5 75.565) (end 189.865 74.93) (width 0.3048) (layer F.Cu) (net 7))
 (segment (start 189.865 74.93) (end 189.9793 75.0443) (width 0.3048) (layer B.Cu) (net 7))
 (segment (start 195.4276 75.0443) (end 189.9793 75.0443) (width 0.3048) (layer B.Cu) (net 7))
 (segment (start 205.74 91.44) (end 206.375 90.805) (width 0.3048) (layer F.Cu) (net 7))
 (segment (start 206.95158 90.805) (end 206.375 90.805) (width 0.3048) (layer F.Cu) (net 7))
 (segment (start 195.4276 72.2757) (end 194.4243 72.2757) (width 0.3048) (layer F.Cu) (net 8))
 (segment (start 205.74 89.535) (end 205.105 90.17) (width 0.3048) (layer F.Cu) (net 8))
 (segment (start 205.105 90.17) (end 195.58 90.17) (width 0.3048) (layer F.Cu) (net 8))
 (segment (start 195.58 90.17) (end 192.405 86.995) (width 0.3048) (layer F.Cu) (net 8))
 (segment (start 192.405 86.995) (end 192.405 74.295) (width 0.3048) (layer F.Cu) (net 8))
 (segment (start 192.405 74.295) (end 194.31 72.39) (width 0.3048) (layer F.Cu) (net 8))
 (segment (start 205.74 89.535) (end 206.95158 89.535) (width 0.3048) (layer F.Cu) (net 8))
 (segment (start 194.4243 72.2757) (end 194.31 72.39) (width 0.3048) (layer F.Cu) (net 8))
 (segment (start 206.85 99.695) (end 207.645 99.695) (width 0.3048) (layer F.Cu) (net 10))
 (segment (start 208.28 100.33) (end 206.28 100.33) (width 0.3048) (layer B.Cu) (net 10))
 (via (at 208.28 100.33) (size 0.6) (drill 0.4) (layers F.Cu B.Cu) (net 10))
 (segment (start 207.645 99.695) (end 208.28 100.33) (width 0.3048) (layer F.Cu) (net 10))
 (segment (start 190.5 100.33) (end 191.135 100.33) (width 0.3048) (layer F.Cu) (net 10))
 (segment (start 191.135 100.33) (end 191.77 99.695) (width 0.3048) (layer F.Cu) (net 10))
 (segment (start 191.77 99.695) (end 206.85 99.695) (width 0.3048) (layer F.Cu) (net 10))
 (segment (start 206.85 98.425) (end 207.645 98.425) (width 0.3048) (layer F.Cu) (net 11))
 (segment (start 208.28 97.79) (end 206.28 97.79) (width 0.3048) (layer B.Cu) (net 11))
 (via (at 208.28 97.79) (size 0.6) (drill 0.4) (layers F.Cu B.Cu) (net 11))
 (segment (start 207.645 98.425) (end 208.28 97.79) (width 0.3048) (layer F.Cu) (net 11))
 (segment (start 190.5 97.79) (end 191.135 97.79) (width 0.3048) (layer F.Cu) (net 11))
 (segment (start 191.135 97.79) (end 191.77 98.425) (width 0.3048) (layer F.Cu) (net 11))
 (segment (start 191.77 98.425) (end 206.85 98.425) (width 0.3048) (layer F.Cu) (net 11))
 (segment (start 210.28 99.06) (end 208.28 99.06) (width 0.3048) (layer B.Cu) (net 12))
 (segment (start 207.485 96.52) (end 206.85 97.155) (width 0.3048) (layer F.Cu) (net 12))
 (segment (start 208.915 96.52) (end 207.485 96.52) (width 0.3048) (layer F.Cu) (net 12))
 (segment (start 209.55 97.155) (end 208.915 96.52) (width 0.3048) (layer F.Cu) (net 12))
 (segment (start 209.55 97.79) (end 209.55 97.155) (width 0.3048) (layer F.Cu) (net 12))
 (segment (start 208.28 99.06) (end 209.55 97.79) (width 0.3048) (layer F.Cu) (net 12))
 (via (at 208.28 99.06) (size 0.6) (drill 0.4) (layers F.Cu B.Cu) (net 12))
 (segment (start 210.28 100.33) (end 210.28 99.06) (width 0.3048) (layer B.Cu) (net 12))
 (segment (start 210.28 99.06) (end 210.28 97.79) (width 0.3048) (layer B.Cu) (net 12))
 (segment (start 212.25 100.965) (end 217.17 100.965) (width 0.3048) (layer F.Cu) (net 13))
 (segment (start 217.805 100.33) (end 220.345 100.33) (width 0.3048) (layer F.Cu) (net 13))
 (segment (start 217.17 100.965) (end 217.805 100.33) (width 0.3048) (layer F.Cu) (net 13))
 (segment (start 212.25 97.155) (end 217.17 97.155) (width 0.3048) (layer F.Cu) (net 15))
 (segment (start 217.805 97.79) (end 220.345 97.79) (width 0.3048) (layer F.Cu) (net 15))
 (segment (start 217.17 97.155) (end 217.805 97.79) (width 0.3048) (layer F.Cu) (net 15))
 (via (at 213.995 92.71) (size 1.27) (drill 0.7112) (layers F.Cu B.Cu) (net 22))
 (segment (start 220.345 107.95) (end 218.44 107.95) (width 0.3048) (layer B.Cu) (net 22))
 (segment (start 215.265 104.775) (end 218.44 107.95) (width 0.3048) (layer B.Cu) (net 22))
 (segment (start 215.265 93.98) (end 215.265 104.775) (width 0.3048) (layer B.Cu) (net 22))
 (segment (start 213.995 92.71) (end 215.265 93.98) (width 0.3048) (layer B.Cu) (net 22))
 (segment (start 213.995 92.075) (end 213.995 92.71) (width 0.3048) (layer F.Cu) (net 22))
 (segment (start 213.995 92.075) (end 212.725 90.805) (width 0.3048) (layer F.Cu) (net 22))
 (segment (start 212.14842 90.805) (end 212.725 90.805) (width 0.3048) (layer F.Cu) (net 22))
 (via (at 213.995 95.885) (size 1.27) (drill 0.7112) (layers F.Cu B.Cu) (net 23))
 (segment (start 217.17 110.49) (end 213.995 107.95) (width 0.3048) (layer B.Cu) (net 23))
 (segment (start 213.995 107.95) (end 213.995 95.885) (width 0.3048) (layer B.Cu) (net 23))
 (segment (start 213.995 95.885) (end 215.9 93.98) (width 0.3048) (layer F.Cu) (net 23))
 (segment (start 215.9 93.98) (end 215.9 90.17) (width 0.3048) (layer F.Cu) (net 23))
 (segment (start 215.9 90.17) (end 215.265 89.535) (width 0.3048) (layer F.Cu) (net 23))
 (segment (start 212.14842 89.535) (end 215.265 89.535) (width 0.3048) (layer F.Cu) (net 23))
 (segment (start 217.17 110.49) (end 220.345 110.49) (width 0.3048) (layer B.Cu) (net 23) (status 800000))
 (segment (start 212.14842 88.265) (end 215.9 88.265) (width 0.3048) (layer F.Cu) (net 24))
 (segment (start 218.44 95.25) (end 220.345 95.25) (width 0.3048) (layer F.Cu) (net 24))
 (segment (start 217.17 93.98) (end 218.44 95.25) (width 0.3048) (layer F.Cu) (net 24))
 (segment (start 217.17 89.535) (end 217.17 93.98) (width 0.3048) (layer F.Cu) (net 24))
 (segment (start 215.9 88.265) (end 217.17 89.535) (width 0.3048) (layer F.Cu) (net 24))
 (segment (start 220.345 92.71) (end 219.075 92.71) (width 0.3048) (layer F.Cu) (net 25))
 (segment (start 216.535 86.995) (end 212.14842 86.995) (width 0.3048) (layer F.Cu) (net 25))
 (segment (start 218.44 88.9) (end 216.535 86.995) (width 0.3048) (layer F.Cu) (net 25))
 (segment (start 218.44 92.075) (end 218.44 88.9) (width 0.3048) (layer F.Cu) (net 25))
 (segment (start 219.075 92.71) (end 218.44 92.075) (width 0.3048) (layer F.Cu) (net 25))
 (segment (start 211.55 79.375) (end 213.995 79.375) (width 0.3048) (layer F.Cu) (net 26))
 (segment (start 212.14842 81.915) (end 213.36 81.915) (width 0.3048) (layer F.Cu) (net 26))
 (segment (start 218.44 64.77) (end 220.345 64.77) (width 0.3048) (layer F.Cu) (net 26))
 (segment (start 213.995 69.215) (end 218.44 64.77) (width 0.3048) (layer F.Cu) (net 26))
 (segment (start 213.995 81.28) (end 213.995 79.375) (width 0.3048) (layer F.Cu) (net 26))
 (segment (start 213.995 79.375) (end 213.995 69.215) (width 0.3048) (layer F.Cu) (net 26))
 (segment (start 213.36 81.915) (end 213.995 81.28) (width 0.3048) (layer F.Cu) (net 26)))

